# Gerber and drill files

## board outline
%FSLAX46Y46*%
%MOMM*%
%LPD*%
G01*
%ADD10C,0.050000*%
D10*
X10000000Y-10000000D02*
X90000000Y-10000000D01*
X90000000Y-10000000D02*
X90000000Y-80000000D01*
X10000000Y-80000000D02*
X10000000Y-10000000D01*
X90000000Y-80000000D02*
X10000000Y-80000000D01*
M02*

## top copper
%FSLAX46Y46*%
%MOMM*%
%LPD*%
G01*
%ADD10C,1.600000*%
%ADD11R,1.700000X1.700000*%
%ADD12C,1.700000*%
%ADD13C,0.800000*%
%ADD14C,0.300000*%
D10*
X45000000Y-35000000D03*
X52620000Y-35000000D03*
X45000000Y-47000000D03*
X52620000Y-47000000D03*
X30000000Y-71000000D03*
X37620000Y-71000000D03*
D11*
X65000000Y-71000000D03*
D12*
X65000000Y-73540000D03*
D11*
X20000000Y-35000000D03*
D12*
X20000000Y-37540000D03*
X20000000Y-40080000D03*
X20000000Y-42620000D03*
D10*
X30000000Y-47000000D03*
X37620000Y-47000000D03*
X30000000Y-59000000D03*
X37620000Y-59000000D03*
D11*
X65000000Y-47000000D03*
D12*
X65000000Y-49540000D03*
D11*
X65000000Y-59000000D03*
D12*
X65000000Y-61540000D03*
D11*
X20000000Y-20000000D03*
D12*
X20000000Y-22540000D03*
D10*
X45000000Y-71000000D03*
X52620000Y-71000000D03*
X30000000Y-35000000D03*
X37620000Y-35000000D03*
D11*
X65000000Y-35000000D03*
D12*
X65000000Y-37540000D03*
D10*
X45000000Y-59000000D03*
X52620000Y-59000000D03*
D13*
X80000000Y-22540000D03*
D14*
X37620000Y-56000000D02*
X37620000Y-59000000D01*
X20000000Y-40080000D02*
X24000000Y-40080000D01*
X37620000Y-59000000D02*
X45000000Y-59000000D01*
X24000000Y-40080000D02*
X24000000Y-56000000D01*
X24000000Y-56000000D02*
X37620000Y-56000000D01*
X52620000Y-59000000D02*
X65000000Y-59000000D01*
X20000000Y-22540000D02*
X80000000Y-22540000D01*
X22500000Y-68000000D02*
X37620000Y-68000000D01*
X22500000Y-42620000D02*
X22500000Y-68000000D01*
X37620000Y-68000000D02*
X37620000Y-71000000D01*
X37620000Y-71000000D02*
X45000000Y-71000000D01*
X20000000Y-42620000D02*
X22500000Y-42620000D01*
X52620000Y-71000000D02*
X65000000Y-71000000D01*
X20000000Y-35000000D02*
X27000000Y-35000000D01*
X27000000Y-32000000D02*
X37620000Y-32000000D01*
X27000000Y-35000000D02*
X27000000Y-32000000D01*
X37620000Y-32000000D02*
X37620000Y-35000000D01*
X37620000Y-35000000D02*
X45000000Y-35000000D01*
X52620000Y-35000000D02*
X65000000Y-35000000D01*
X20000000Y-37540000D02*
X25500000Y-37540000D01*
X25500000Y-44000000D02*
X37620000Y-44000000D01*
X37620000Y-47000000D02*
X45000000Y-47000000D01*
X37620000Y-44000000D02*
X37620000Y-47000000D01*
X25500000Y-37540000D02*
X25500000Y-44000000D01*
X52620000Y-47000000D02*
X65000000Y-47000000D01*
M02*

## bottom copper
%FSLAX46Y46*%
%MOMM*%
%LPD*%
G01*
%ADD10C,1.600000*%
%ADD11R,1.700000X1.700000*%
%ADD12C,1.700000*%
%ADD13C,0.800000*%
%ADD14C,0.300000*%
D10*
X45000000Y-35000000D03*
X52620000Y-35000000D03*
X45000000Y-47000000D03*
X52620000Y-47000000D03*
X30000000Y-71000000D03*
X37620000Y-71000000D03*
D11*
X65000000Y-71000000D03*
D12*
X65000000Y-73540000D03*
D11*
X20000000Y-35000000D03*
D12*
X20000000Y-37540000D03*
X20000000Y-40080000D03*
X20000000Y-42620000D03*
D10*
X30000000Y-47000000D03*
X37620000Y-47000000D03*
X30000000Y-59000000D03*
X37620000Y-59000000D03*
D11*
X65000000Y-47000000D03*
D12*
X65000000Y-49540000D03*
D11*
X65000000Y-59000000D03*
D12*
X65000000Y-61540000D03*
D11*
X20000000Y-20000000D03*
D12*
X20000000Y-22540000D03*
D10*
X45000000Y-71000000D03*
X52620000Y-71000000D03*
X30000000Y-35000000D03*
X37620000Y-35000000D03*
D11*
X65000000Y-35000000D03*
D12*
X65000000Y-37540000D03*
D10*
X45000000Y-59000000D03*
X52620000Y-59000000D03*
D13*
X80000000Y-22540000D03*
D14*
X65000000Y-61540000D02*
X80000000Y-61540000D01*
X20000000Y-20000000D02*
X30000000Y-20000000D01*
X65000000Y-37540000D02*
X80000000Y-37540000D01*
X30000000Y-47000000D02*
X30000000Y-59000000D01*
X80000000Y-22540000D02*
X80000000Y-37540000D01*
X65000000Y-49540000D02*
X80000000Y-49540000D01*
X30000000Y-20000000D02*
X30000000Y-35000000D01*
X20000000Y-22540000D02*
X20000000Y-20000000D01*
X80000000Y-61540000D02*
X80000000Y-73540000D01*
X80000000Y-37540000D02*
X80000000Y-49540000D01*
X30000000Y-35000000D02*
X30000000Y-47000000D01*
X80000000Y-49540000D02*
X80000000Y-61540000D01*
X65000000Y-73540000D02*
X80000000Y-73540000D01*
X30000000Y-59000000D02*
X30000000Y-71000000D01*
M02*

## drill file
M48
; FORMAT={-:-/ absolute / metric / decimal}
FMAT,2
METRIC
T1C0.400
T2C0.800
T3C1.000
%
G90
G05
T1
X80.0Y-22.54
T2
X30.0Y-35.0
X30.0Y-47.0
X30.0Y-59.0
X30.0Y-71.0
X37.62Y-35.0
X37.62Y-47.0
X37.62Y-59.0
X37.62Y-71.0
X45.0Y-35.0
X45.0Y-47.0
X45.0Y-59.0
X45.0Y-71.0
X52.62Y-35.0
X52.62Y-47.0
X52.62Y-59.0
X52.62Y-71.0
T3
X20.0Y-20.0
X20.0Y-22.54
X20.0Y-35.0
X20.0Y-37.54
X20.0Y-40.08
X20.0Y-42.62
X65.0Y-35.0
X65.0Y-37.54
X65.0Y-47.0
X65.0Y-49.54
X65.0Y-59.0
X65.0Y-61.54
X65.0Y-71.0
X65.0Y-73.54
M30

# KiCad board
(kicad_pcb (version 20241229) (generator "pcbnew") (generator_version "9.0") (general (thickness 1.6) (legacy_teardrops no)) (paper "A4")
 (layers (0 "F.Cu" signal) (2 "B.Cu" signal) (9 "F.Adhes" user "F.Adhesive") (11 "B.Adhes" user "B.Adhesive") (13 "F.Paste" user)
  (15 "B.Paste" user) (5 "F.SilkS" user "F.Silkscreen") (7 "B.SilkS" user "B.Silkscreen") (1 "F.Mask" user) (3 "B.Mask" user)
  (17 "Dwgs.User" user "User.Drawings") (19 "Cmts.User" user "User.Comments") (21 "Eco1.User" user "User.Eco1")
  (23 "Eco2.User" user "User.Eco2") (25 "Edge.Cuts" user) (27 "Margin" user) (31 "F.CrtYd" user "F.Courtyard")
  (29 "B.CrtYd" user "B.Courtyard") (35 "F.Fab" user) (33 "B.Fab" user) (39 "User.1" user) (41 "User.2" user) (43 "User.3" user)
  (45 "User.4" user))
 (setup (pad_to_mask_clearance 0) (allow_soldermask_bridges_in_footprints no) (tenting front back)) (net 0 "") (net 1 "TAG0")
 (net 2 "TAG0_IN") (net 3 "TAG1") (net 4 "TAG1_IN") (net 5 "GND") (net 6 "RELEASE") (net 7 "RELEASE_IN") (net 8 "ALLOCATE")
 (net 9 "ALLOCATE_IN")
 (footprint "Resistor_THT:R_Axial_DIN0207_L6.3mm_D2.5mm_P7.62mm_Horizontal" (layer "F.Cu") (at 45 35)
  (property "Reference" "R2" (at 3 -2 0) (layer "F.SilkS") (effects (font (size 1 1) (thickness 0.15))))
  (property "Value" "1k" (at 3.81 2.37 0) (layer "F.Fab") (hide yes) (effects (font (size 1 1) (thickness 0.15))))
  (pad "1" thru_hole circle (at 0 0) (size 1.6 1.6) (drill 0.8) (layers "*.Cu" "*.Mask") (remove_unused_layers no) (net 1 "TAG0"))
  (pad "2" thru_hole circle (at 7.62 0) (size 1.6 1.6) (drill 0.8) (layers "*.Cu" "*.Mask") (remove_unused_layers no) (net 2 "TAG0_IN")))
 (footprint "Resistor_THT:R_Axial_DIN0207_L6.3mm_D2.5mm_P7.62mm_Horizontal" (layer "F.Cu") (at 45 47)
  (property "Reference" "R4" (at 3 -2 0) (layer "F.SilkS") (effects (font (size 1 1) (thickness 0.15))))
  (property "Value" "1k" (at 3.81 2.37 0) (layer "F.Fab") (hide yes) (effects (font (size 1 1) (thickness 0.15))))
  (pad "1" thru_hole circle (at 0 0) (size 1.6 1.6) (drill 0.8) (layers "*.Cu" "*.Mask") (remove_unused_layers no) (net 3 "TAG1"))
  (pad "2" thru_hole circle (at 7.62 0) (size 1.6 1.6) (drill 0.8) (layers "*.Cu" "*.Mask") (remove_unused_layers no) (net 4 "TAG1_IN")))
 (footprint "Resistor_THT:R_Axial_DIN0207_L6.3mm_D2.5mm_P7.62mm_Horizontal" (layer "F.Cu") (at 30 71)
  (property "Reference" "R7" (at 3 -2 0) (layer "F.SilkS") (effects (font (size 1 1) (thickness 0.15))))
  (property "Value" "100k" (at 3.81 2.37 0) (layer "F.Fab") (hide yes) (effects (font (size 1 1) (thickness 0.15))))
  (pad "1" thru_hole circle (at 0 0) (size 1.6 1.6) (drill 0.8) (layers "*.Cu" "*.Mask") (remove_unused_layers no) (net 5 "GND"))
  (pad "2" thru_hole circle (at 7.62 0) (size 1.6 1.6) (drill 0.8) (layers "*.Cu" "*.Mask") (remove_unused_layers no) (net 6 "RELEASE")))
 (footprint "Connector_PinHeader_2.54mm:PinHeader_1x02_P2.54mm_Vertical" (layer "F.Cu") (at 65 71)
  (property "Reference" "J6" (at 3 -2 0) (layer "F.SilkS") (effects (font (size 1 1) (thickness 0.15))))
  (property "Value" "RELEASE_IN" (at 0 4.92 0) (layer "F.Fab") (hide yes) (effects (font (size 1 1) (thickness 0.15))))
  (pad "1" thru_hole rect (at 0 0) (size 1.7 1.7) (drill 1) (layers "*.Cu" "*.Mask") (remove_unused_layers no) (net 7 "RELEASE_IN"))
  (pad "2" thru_hole circle (at 0 2.54) (size 1.7 1.7) (drill 1) (layers "*.Cu" "*.Mask") (remove_unused_layers no) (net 5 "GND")))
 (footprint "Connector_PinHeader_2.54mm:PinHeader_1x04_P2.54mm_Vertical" (layer "F.Cu") (at 20 35)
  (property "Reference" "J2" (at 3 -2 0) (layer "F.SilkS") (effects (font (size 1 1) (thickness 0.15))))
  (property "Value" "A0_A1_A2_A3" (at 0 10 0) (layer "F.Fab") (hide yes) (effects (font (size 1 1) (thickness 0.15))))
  (pad "1" thru_hole rect (at 0 0) (size 1.7 1.7) (drill 1) (layers "*.Cu" "*.Mask") (remove_unused_layers no) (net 1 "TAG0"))
  (pad "2" thru_hole circle (at 0 2.54) (size 1.7 1.7) (drill 1) (layers "*.Cu" "*.Mask") (remove_unused_layers no) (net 3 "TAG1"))
  (pad "3" thru_hole circle (at 0 5.08) (size 1.7 1.7) (drill 1) (layers "*.Cu" "*.Mask") (remove_unused_layers no) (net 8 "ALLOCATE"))
  (pad "4" thru_hole circle (at 0 7.62) (size 1.7 1.7) (drill 1) (layers "*.Cu" "*.Mask") (remove_unused_layers no) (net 6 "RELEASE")))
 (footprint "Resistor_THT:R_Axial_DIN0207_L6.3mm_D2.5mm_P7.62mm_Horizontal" (layer "F.Cu") (at 30 47)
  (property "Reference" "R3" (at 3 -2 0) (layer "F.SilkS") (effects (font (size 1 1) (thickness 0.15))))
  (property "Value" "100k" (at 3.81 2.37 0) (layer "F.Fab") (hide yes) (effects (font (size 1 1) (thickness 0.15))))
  (pad "1" thru_hole circle (at 0 0) (size 1.6 1.6) (drill 0.8) (layers "*.Cu" "*.Mask") (remove_unused_layers no) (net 5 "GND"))
  (pad "2" thru_hole circle (at 7.62 0) (size 1.6 1.6) (drill 0.8) (layers "*.Cu" "*.Mask") (remove_unused_layers no) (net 3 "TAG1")))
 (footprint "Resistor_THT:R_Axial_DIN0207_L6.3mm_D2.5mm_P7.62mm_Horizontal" (layer "F.Cu") (at 30 59)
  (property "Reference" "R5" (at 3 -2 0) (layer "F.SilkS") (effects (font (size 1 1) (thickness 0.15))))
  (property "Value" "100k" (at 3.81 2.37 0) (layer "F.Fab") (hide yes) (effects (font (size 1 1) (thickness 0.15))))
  (pad "1" thru_hole circle (at 0 0) (size 1.6 1.6) (drill 0.8) (layers "*.Cu" "*.Mask") (remove_unused_layers no) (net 5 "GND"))
  (pad "2" thru_hole circle (at 7.62 0) (size 1.6 1.6) (drill 0.8) (layers "*.Cu" "*.Mask") (remove_unused_layers no) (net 8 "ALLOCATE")))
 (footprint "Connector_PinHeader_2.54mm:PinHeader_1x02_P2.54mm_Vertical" (layer "F.Cu") (at 65 47)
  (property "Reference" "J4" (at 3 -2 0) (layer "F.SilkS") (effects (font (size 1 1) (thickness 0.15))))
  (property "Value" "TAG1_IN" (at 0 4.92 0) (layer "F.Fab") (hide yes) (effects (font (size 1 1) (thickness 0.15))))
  (pad "1" thru_hole rect (at 0 0) (size 1.7 1.7) (drill 1) (layers "*.Cu" "*.Mask") (remove_unused_layers no) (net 4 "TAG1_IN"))
  (pad "2" thru_hole circle (at 0 2.54) (size 1.7 1.7) (drill 1) (layers "*.Cu" "*.Mask") (remove_unused_layers no) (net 5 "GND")))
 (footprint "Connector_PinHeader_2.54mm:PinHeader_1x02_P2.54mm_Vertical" (layer "F.Cu") (at 65 59)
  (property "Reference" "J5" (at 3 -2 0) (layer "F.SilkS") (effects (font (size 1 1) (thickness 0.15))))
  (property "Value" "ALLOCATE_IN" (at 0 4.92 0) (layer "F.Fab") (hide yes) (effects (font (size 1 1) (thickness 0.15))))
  (pad "1" thru_hole rect (at 0 0) (size 1.7 1.7) (drill 1) (layers "*.Cu" "*.Mask") (remove_unused_layers no) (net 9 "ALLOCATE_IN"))
  (pad "2" thru_hole circle (at 0 2.54) (size 1.7 1.7) (drill 1) (layers "*.Cu" "*.Mask") (remove_unused_layers no) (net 5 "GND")))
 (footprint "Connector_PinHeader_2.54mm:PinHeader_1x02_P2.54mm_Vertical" (layer "F.Cu") (at 20 20)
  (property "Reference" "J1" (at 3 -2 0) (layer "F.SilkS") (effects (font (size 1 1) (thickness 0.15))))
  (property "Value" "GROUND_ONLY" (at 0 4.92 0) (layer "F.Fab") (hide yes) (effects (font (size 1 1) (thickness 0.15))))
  (pad "1" thru_hole rect (at 0 0) (size 1.7 1.7) (drill 1) (layers "*.Cu" "*.Mask") (remove_unused_layers no) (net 5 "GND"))
  (pad "2" thru_hole circle (at 0 2.54) (size 1.7 1.7) (drill 1) (layers "*.Cu" "*.Mask") (remove_unused_layers no) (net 5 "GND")))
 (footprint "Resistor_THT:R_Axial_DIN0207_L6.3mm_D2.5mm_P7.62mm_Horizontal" (layer "F.Cu") (at 45 71)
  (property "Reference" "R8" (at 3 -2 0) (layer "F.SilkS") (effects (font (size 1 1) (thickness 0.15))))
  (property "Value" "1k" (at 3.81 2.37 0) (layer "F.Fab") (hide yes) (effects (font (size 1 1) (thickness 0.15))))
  (pad "1" thru_hole circle (at 0 0) (size 1.6 1.6) (drill 0.8) (layers "*.Cu" "*.Mask") (remove_unused_layers no) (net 6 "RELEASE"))
  (pad "2" thru_hole circle (at 7.62 0) (size 1.6 1.6) (drill 0.8) (layers "*.Cu" "*.Mask") (remove_unused_layers no) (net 7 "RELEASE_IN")))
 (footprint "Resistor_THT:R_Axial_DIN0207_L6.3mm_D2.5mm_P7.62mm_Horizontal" (layer "F.Cu") (at 30 35)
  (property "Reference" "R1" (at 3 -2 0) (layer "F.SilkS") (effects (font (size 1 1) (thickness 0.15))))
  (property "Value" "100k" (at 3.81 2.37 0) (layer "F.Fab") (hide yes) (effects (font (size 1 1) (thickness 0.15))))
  (pad "1" thru_hole circle (at 0 0) (size 1.6 1.6) (drill 0.8) (layers "*.Cu" "*.Mask") (remove_unused_layers no) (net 5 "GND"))
  (pad "2" thru_hole circle (at 7.62 0) (size 1.6 1.6) (drill 0.8) (layers "*.Cu" "*.Mask") (remove_unused_layers no) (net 1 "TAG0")))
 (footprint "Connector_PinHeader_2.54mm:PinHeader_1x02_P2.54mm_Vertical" (layer "F.Cu") (at 65 35)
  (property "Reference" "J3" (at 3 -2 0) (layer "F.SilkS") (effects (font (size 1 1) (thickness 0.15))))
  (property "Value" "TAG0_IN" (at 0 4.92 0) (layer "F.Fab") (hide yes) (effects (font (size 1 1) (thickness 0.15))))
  (pad "1" thru_hole rect (at 0 0) (size 1.7 1.7) (drill 1) (layers "*.Cu" "*.Mask") (remove_unused_layers no) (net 2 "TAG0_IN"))
  (pad "2" thru_hole circle (at 0 2.54) (size 1.7 1.7) (drill 1) (layers "*.Cu" "*.Mask") (remove_unused_layers no) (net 5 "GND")))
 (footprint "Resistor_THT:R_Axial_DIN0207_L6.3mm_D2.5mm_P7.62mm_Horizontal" (layer "F.Cu") (at 45 59)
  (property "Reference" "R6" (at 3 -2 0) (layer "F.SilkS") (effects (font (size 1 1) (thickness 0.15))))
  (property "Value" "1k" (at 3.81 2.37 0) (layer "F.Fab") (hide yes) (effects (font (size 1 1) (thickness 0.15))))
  (pad "1" thru_hole circle (at 0 0) (size 1.6 1.6) (drill 0.8) (layers "*.Cu" "*.Mask") (remove_unused_layers no) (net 8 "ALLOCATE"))
  (pad "2" thru_hole circle (at 7.62 0) (size 1.6 1.6) (drill 0.8) (layers "*.Cu" "*.Mask") (remove_unused_layers no) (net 9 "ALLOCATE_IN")))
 (gr_line (start 10 10) (end 90 10) (stroke (width 0.05) (type default)) (layer "Edge.Cuts"))
 (gr_line (start 90 10) (end 90 80) (stroke (width 0.05) (type default)) (layer "Edge.Cuts"))
 (gr_line (start 10 80) (end 10 10) (stroke (width 0.05) (type default)) (layer "Edge.Cuts"))
 (gr_line (start 90 80) (end 10 80) (stroke (width 0.05) (type default)) (layer "Edge.Cuts"))
 (segment (start 37.62 56) (end 37.62 59) (width 0.3) (layer "F.Cu") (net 8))
 (segment (start 20 40.08) (end 24 40.08) (width 0.3) (layer "F.Cu") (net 8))
 (segment (start 37.62 59) (end 45 59) (width 0.3) (layer "F.Cu") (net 8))
 (segment (start 24 40.08) (end 24 56) (width 0.3) (layer "F.Cu") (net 8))
 (segment (start 24 56) (end 37.62 56) (width 0.3) (layer "F.Cu") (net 8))
 (segment (start 52.62 59) (end 65 59) (width 0.3) (layer "F.Cu") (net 9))
 (segment (start 20 22.54) (end 80 22.54) (width 0.3) (layer "F.Cu") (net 5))
 (via (at 80 22.54) (size 0.8) (drill 0.4) (layers "F.Cu" "B.Cu") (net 5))
 (segment (start 65 61.54) (end 80 61.54) (width 0.3) (layer "B.Cu") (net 5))
 (segment (start 20 20) (end 30 20) (width 0.3) (layer "B.Cu") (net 5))
 (segment (start 65 37.54) (end 80 37.54) (width 0.3) (layer "B.Cu") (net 5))
 (segment (start 30 47) (end 30 59) (width 0.3) (layer "B.Cu") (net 5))
 (segment (start 80 22.54) (end 80 37.54) (width 0.3) (layer "B.Cu") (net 5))
 (segment (start 65 49.54) (end 80 49.54) (width 0.3) (layer "B.Cu") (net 5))
 (segment (start 30 20) (end 30 35) (width 0.3) (layer "B.Cu") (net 5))
 (segment (start 20 22.54) (end 20 20) (width 0.3) (layer "B.Cu") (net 5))
 (segment (start 80 61.54) (end 80 73.54) (width 0.3) (layer "B.Cu") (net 5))
 (segment (start 80 37.54) (end 80 49.54) (width 0.3) (layer "B.Cu") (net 5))
 (segment (start 30 35) (end 30 47) (width 0.3) (layer "B.Cu") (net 5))
 (segment (start 80 49.54) (end 80 61.54) (width 0.3) (layer "B.Cu") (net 5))
 (segment (start 65 73.54) (end 80 73.54) (width 0.3) (layer "B.Cu") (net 5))
 (segment (start 30 59) (end 30 71) (width 0.3) (layer "B.Cu") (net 5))
 (segment (start 22.5 68) (end 37.62 68) (width 0.3) (layer "F.Cu") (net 6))
 (segment (start 22.5 42.62) (end 22.5 68) (width 0.3) (layer "F.Cu") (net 6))
 (segment (start 37.62 68) (end 37.62 71) (width 0.3) (layer "F.Cu") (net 6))
 (segment (start 37.62 71) (end 45 71) (width 0.3) (layer "F.Cu") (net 6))
 (segment (start 20 42.62) (end 22.5 42.62) (width 0.3) (layer "F.Cu") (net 6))
 (segment (start 52.62 71) (end 65 71) (width 0.3) (layer "F.Cu") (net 7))
 (segment (start 20 35) (end 27 35) (width 0.3) (layer "F.Cu") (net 1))
 (segment (start 27 32) (end 37.62 32) (width 0.3) (layer "F.Cu") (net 1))
 (segment (start 27 35) (end 27 32) (width 0.3) (layer "F.Cu") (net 1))
 (segment (start 37.62 32) (end 37.62 35) (width 0.3) (layer "F.Cu") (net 1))
 (segment (start 37.62 35) (end 45 35) (width 0.3) (layer "F.Cu") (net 1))
 (segment (start 52.62 35) (end 65 35) (width 0.3) (layer "F.Cu") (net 2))
 (segment (start 20 37.54) (end 25.5 37.54) (width 0.3) (layer "F.Cu") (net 3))
 (segment (start 25.5 44) (end 37.62 44) (width 0.3) (layer "F.Cu") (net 3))
 (segment (start 37.62 47) (end 45 47) (width 0.3) (layer "F.Cu") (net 3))
 (segment (start 37.62 44) (end 37.62 47) (width 0.3) (layer "F.Cu") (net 3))
 (segment (start 25.5 37.54) (end 25.5 44) (width 0.3) (layer "F.Cu") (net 3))
 (segment (start 52.62 47) (end 65 47) (width 0.3) (layer "F.Cu") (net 4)))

